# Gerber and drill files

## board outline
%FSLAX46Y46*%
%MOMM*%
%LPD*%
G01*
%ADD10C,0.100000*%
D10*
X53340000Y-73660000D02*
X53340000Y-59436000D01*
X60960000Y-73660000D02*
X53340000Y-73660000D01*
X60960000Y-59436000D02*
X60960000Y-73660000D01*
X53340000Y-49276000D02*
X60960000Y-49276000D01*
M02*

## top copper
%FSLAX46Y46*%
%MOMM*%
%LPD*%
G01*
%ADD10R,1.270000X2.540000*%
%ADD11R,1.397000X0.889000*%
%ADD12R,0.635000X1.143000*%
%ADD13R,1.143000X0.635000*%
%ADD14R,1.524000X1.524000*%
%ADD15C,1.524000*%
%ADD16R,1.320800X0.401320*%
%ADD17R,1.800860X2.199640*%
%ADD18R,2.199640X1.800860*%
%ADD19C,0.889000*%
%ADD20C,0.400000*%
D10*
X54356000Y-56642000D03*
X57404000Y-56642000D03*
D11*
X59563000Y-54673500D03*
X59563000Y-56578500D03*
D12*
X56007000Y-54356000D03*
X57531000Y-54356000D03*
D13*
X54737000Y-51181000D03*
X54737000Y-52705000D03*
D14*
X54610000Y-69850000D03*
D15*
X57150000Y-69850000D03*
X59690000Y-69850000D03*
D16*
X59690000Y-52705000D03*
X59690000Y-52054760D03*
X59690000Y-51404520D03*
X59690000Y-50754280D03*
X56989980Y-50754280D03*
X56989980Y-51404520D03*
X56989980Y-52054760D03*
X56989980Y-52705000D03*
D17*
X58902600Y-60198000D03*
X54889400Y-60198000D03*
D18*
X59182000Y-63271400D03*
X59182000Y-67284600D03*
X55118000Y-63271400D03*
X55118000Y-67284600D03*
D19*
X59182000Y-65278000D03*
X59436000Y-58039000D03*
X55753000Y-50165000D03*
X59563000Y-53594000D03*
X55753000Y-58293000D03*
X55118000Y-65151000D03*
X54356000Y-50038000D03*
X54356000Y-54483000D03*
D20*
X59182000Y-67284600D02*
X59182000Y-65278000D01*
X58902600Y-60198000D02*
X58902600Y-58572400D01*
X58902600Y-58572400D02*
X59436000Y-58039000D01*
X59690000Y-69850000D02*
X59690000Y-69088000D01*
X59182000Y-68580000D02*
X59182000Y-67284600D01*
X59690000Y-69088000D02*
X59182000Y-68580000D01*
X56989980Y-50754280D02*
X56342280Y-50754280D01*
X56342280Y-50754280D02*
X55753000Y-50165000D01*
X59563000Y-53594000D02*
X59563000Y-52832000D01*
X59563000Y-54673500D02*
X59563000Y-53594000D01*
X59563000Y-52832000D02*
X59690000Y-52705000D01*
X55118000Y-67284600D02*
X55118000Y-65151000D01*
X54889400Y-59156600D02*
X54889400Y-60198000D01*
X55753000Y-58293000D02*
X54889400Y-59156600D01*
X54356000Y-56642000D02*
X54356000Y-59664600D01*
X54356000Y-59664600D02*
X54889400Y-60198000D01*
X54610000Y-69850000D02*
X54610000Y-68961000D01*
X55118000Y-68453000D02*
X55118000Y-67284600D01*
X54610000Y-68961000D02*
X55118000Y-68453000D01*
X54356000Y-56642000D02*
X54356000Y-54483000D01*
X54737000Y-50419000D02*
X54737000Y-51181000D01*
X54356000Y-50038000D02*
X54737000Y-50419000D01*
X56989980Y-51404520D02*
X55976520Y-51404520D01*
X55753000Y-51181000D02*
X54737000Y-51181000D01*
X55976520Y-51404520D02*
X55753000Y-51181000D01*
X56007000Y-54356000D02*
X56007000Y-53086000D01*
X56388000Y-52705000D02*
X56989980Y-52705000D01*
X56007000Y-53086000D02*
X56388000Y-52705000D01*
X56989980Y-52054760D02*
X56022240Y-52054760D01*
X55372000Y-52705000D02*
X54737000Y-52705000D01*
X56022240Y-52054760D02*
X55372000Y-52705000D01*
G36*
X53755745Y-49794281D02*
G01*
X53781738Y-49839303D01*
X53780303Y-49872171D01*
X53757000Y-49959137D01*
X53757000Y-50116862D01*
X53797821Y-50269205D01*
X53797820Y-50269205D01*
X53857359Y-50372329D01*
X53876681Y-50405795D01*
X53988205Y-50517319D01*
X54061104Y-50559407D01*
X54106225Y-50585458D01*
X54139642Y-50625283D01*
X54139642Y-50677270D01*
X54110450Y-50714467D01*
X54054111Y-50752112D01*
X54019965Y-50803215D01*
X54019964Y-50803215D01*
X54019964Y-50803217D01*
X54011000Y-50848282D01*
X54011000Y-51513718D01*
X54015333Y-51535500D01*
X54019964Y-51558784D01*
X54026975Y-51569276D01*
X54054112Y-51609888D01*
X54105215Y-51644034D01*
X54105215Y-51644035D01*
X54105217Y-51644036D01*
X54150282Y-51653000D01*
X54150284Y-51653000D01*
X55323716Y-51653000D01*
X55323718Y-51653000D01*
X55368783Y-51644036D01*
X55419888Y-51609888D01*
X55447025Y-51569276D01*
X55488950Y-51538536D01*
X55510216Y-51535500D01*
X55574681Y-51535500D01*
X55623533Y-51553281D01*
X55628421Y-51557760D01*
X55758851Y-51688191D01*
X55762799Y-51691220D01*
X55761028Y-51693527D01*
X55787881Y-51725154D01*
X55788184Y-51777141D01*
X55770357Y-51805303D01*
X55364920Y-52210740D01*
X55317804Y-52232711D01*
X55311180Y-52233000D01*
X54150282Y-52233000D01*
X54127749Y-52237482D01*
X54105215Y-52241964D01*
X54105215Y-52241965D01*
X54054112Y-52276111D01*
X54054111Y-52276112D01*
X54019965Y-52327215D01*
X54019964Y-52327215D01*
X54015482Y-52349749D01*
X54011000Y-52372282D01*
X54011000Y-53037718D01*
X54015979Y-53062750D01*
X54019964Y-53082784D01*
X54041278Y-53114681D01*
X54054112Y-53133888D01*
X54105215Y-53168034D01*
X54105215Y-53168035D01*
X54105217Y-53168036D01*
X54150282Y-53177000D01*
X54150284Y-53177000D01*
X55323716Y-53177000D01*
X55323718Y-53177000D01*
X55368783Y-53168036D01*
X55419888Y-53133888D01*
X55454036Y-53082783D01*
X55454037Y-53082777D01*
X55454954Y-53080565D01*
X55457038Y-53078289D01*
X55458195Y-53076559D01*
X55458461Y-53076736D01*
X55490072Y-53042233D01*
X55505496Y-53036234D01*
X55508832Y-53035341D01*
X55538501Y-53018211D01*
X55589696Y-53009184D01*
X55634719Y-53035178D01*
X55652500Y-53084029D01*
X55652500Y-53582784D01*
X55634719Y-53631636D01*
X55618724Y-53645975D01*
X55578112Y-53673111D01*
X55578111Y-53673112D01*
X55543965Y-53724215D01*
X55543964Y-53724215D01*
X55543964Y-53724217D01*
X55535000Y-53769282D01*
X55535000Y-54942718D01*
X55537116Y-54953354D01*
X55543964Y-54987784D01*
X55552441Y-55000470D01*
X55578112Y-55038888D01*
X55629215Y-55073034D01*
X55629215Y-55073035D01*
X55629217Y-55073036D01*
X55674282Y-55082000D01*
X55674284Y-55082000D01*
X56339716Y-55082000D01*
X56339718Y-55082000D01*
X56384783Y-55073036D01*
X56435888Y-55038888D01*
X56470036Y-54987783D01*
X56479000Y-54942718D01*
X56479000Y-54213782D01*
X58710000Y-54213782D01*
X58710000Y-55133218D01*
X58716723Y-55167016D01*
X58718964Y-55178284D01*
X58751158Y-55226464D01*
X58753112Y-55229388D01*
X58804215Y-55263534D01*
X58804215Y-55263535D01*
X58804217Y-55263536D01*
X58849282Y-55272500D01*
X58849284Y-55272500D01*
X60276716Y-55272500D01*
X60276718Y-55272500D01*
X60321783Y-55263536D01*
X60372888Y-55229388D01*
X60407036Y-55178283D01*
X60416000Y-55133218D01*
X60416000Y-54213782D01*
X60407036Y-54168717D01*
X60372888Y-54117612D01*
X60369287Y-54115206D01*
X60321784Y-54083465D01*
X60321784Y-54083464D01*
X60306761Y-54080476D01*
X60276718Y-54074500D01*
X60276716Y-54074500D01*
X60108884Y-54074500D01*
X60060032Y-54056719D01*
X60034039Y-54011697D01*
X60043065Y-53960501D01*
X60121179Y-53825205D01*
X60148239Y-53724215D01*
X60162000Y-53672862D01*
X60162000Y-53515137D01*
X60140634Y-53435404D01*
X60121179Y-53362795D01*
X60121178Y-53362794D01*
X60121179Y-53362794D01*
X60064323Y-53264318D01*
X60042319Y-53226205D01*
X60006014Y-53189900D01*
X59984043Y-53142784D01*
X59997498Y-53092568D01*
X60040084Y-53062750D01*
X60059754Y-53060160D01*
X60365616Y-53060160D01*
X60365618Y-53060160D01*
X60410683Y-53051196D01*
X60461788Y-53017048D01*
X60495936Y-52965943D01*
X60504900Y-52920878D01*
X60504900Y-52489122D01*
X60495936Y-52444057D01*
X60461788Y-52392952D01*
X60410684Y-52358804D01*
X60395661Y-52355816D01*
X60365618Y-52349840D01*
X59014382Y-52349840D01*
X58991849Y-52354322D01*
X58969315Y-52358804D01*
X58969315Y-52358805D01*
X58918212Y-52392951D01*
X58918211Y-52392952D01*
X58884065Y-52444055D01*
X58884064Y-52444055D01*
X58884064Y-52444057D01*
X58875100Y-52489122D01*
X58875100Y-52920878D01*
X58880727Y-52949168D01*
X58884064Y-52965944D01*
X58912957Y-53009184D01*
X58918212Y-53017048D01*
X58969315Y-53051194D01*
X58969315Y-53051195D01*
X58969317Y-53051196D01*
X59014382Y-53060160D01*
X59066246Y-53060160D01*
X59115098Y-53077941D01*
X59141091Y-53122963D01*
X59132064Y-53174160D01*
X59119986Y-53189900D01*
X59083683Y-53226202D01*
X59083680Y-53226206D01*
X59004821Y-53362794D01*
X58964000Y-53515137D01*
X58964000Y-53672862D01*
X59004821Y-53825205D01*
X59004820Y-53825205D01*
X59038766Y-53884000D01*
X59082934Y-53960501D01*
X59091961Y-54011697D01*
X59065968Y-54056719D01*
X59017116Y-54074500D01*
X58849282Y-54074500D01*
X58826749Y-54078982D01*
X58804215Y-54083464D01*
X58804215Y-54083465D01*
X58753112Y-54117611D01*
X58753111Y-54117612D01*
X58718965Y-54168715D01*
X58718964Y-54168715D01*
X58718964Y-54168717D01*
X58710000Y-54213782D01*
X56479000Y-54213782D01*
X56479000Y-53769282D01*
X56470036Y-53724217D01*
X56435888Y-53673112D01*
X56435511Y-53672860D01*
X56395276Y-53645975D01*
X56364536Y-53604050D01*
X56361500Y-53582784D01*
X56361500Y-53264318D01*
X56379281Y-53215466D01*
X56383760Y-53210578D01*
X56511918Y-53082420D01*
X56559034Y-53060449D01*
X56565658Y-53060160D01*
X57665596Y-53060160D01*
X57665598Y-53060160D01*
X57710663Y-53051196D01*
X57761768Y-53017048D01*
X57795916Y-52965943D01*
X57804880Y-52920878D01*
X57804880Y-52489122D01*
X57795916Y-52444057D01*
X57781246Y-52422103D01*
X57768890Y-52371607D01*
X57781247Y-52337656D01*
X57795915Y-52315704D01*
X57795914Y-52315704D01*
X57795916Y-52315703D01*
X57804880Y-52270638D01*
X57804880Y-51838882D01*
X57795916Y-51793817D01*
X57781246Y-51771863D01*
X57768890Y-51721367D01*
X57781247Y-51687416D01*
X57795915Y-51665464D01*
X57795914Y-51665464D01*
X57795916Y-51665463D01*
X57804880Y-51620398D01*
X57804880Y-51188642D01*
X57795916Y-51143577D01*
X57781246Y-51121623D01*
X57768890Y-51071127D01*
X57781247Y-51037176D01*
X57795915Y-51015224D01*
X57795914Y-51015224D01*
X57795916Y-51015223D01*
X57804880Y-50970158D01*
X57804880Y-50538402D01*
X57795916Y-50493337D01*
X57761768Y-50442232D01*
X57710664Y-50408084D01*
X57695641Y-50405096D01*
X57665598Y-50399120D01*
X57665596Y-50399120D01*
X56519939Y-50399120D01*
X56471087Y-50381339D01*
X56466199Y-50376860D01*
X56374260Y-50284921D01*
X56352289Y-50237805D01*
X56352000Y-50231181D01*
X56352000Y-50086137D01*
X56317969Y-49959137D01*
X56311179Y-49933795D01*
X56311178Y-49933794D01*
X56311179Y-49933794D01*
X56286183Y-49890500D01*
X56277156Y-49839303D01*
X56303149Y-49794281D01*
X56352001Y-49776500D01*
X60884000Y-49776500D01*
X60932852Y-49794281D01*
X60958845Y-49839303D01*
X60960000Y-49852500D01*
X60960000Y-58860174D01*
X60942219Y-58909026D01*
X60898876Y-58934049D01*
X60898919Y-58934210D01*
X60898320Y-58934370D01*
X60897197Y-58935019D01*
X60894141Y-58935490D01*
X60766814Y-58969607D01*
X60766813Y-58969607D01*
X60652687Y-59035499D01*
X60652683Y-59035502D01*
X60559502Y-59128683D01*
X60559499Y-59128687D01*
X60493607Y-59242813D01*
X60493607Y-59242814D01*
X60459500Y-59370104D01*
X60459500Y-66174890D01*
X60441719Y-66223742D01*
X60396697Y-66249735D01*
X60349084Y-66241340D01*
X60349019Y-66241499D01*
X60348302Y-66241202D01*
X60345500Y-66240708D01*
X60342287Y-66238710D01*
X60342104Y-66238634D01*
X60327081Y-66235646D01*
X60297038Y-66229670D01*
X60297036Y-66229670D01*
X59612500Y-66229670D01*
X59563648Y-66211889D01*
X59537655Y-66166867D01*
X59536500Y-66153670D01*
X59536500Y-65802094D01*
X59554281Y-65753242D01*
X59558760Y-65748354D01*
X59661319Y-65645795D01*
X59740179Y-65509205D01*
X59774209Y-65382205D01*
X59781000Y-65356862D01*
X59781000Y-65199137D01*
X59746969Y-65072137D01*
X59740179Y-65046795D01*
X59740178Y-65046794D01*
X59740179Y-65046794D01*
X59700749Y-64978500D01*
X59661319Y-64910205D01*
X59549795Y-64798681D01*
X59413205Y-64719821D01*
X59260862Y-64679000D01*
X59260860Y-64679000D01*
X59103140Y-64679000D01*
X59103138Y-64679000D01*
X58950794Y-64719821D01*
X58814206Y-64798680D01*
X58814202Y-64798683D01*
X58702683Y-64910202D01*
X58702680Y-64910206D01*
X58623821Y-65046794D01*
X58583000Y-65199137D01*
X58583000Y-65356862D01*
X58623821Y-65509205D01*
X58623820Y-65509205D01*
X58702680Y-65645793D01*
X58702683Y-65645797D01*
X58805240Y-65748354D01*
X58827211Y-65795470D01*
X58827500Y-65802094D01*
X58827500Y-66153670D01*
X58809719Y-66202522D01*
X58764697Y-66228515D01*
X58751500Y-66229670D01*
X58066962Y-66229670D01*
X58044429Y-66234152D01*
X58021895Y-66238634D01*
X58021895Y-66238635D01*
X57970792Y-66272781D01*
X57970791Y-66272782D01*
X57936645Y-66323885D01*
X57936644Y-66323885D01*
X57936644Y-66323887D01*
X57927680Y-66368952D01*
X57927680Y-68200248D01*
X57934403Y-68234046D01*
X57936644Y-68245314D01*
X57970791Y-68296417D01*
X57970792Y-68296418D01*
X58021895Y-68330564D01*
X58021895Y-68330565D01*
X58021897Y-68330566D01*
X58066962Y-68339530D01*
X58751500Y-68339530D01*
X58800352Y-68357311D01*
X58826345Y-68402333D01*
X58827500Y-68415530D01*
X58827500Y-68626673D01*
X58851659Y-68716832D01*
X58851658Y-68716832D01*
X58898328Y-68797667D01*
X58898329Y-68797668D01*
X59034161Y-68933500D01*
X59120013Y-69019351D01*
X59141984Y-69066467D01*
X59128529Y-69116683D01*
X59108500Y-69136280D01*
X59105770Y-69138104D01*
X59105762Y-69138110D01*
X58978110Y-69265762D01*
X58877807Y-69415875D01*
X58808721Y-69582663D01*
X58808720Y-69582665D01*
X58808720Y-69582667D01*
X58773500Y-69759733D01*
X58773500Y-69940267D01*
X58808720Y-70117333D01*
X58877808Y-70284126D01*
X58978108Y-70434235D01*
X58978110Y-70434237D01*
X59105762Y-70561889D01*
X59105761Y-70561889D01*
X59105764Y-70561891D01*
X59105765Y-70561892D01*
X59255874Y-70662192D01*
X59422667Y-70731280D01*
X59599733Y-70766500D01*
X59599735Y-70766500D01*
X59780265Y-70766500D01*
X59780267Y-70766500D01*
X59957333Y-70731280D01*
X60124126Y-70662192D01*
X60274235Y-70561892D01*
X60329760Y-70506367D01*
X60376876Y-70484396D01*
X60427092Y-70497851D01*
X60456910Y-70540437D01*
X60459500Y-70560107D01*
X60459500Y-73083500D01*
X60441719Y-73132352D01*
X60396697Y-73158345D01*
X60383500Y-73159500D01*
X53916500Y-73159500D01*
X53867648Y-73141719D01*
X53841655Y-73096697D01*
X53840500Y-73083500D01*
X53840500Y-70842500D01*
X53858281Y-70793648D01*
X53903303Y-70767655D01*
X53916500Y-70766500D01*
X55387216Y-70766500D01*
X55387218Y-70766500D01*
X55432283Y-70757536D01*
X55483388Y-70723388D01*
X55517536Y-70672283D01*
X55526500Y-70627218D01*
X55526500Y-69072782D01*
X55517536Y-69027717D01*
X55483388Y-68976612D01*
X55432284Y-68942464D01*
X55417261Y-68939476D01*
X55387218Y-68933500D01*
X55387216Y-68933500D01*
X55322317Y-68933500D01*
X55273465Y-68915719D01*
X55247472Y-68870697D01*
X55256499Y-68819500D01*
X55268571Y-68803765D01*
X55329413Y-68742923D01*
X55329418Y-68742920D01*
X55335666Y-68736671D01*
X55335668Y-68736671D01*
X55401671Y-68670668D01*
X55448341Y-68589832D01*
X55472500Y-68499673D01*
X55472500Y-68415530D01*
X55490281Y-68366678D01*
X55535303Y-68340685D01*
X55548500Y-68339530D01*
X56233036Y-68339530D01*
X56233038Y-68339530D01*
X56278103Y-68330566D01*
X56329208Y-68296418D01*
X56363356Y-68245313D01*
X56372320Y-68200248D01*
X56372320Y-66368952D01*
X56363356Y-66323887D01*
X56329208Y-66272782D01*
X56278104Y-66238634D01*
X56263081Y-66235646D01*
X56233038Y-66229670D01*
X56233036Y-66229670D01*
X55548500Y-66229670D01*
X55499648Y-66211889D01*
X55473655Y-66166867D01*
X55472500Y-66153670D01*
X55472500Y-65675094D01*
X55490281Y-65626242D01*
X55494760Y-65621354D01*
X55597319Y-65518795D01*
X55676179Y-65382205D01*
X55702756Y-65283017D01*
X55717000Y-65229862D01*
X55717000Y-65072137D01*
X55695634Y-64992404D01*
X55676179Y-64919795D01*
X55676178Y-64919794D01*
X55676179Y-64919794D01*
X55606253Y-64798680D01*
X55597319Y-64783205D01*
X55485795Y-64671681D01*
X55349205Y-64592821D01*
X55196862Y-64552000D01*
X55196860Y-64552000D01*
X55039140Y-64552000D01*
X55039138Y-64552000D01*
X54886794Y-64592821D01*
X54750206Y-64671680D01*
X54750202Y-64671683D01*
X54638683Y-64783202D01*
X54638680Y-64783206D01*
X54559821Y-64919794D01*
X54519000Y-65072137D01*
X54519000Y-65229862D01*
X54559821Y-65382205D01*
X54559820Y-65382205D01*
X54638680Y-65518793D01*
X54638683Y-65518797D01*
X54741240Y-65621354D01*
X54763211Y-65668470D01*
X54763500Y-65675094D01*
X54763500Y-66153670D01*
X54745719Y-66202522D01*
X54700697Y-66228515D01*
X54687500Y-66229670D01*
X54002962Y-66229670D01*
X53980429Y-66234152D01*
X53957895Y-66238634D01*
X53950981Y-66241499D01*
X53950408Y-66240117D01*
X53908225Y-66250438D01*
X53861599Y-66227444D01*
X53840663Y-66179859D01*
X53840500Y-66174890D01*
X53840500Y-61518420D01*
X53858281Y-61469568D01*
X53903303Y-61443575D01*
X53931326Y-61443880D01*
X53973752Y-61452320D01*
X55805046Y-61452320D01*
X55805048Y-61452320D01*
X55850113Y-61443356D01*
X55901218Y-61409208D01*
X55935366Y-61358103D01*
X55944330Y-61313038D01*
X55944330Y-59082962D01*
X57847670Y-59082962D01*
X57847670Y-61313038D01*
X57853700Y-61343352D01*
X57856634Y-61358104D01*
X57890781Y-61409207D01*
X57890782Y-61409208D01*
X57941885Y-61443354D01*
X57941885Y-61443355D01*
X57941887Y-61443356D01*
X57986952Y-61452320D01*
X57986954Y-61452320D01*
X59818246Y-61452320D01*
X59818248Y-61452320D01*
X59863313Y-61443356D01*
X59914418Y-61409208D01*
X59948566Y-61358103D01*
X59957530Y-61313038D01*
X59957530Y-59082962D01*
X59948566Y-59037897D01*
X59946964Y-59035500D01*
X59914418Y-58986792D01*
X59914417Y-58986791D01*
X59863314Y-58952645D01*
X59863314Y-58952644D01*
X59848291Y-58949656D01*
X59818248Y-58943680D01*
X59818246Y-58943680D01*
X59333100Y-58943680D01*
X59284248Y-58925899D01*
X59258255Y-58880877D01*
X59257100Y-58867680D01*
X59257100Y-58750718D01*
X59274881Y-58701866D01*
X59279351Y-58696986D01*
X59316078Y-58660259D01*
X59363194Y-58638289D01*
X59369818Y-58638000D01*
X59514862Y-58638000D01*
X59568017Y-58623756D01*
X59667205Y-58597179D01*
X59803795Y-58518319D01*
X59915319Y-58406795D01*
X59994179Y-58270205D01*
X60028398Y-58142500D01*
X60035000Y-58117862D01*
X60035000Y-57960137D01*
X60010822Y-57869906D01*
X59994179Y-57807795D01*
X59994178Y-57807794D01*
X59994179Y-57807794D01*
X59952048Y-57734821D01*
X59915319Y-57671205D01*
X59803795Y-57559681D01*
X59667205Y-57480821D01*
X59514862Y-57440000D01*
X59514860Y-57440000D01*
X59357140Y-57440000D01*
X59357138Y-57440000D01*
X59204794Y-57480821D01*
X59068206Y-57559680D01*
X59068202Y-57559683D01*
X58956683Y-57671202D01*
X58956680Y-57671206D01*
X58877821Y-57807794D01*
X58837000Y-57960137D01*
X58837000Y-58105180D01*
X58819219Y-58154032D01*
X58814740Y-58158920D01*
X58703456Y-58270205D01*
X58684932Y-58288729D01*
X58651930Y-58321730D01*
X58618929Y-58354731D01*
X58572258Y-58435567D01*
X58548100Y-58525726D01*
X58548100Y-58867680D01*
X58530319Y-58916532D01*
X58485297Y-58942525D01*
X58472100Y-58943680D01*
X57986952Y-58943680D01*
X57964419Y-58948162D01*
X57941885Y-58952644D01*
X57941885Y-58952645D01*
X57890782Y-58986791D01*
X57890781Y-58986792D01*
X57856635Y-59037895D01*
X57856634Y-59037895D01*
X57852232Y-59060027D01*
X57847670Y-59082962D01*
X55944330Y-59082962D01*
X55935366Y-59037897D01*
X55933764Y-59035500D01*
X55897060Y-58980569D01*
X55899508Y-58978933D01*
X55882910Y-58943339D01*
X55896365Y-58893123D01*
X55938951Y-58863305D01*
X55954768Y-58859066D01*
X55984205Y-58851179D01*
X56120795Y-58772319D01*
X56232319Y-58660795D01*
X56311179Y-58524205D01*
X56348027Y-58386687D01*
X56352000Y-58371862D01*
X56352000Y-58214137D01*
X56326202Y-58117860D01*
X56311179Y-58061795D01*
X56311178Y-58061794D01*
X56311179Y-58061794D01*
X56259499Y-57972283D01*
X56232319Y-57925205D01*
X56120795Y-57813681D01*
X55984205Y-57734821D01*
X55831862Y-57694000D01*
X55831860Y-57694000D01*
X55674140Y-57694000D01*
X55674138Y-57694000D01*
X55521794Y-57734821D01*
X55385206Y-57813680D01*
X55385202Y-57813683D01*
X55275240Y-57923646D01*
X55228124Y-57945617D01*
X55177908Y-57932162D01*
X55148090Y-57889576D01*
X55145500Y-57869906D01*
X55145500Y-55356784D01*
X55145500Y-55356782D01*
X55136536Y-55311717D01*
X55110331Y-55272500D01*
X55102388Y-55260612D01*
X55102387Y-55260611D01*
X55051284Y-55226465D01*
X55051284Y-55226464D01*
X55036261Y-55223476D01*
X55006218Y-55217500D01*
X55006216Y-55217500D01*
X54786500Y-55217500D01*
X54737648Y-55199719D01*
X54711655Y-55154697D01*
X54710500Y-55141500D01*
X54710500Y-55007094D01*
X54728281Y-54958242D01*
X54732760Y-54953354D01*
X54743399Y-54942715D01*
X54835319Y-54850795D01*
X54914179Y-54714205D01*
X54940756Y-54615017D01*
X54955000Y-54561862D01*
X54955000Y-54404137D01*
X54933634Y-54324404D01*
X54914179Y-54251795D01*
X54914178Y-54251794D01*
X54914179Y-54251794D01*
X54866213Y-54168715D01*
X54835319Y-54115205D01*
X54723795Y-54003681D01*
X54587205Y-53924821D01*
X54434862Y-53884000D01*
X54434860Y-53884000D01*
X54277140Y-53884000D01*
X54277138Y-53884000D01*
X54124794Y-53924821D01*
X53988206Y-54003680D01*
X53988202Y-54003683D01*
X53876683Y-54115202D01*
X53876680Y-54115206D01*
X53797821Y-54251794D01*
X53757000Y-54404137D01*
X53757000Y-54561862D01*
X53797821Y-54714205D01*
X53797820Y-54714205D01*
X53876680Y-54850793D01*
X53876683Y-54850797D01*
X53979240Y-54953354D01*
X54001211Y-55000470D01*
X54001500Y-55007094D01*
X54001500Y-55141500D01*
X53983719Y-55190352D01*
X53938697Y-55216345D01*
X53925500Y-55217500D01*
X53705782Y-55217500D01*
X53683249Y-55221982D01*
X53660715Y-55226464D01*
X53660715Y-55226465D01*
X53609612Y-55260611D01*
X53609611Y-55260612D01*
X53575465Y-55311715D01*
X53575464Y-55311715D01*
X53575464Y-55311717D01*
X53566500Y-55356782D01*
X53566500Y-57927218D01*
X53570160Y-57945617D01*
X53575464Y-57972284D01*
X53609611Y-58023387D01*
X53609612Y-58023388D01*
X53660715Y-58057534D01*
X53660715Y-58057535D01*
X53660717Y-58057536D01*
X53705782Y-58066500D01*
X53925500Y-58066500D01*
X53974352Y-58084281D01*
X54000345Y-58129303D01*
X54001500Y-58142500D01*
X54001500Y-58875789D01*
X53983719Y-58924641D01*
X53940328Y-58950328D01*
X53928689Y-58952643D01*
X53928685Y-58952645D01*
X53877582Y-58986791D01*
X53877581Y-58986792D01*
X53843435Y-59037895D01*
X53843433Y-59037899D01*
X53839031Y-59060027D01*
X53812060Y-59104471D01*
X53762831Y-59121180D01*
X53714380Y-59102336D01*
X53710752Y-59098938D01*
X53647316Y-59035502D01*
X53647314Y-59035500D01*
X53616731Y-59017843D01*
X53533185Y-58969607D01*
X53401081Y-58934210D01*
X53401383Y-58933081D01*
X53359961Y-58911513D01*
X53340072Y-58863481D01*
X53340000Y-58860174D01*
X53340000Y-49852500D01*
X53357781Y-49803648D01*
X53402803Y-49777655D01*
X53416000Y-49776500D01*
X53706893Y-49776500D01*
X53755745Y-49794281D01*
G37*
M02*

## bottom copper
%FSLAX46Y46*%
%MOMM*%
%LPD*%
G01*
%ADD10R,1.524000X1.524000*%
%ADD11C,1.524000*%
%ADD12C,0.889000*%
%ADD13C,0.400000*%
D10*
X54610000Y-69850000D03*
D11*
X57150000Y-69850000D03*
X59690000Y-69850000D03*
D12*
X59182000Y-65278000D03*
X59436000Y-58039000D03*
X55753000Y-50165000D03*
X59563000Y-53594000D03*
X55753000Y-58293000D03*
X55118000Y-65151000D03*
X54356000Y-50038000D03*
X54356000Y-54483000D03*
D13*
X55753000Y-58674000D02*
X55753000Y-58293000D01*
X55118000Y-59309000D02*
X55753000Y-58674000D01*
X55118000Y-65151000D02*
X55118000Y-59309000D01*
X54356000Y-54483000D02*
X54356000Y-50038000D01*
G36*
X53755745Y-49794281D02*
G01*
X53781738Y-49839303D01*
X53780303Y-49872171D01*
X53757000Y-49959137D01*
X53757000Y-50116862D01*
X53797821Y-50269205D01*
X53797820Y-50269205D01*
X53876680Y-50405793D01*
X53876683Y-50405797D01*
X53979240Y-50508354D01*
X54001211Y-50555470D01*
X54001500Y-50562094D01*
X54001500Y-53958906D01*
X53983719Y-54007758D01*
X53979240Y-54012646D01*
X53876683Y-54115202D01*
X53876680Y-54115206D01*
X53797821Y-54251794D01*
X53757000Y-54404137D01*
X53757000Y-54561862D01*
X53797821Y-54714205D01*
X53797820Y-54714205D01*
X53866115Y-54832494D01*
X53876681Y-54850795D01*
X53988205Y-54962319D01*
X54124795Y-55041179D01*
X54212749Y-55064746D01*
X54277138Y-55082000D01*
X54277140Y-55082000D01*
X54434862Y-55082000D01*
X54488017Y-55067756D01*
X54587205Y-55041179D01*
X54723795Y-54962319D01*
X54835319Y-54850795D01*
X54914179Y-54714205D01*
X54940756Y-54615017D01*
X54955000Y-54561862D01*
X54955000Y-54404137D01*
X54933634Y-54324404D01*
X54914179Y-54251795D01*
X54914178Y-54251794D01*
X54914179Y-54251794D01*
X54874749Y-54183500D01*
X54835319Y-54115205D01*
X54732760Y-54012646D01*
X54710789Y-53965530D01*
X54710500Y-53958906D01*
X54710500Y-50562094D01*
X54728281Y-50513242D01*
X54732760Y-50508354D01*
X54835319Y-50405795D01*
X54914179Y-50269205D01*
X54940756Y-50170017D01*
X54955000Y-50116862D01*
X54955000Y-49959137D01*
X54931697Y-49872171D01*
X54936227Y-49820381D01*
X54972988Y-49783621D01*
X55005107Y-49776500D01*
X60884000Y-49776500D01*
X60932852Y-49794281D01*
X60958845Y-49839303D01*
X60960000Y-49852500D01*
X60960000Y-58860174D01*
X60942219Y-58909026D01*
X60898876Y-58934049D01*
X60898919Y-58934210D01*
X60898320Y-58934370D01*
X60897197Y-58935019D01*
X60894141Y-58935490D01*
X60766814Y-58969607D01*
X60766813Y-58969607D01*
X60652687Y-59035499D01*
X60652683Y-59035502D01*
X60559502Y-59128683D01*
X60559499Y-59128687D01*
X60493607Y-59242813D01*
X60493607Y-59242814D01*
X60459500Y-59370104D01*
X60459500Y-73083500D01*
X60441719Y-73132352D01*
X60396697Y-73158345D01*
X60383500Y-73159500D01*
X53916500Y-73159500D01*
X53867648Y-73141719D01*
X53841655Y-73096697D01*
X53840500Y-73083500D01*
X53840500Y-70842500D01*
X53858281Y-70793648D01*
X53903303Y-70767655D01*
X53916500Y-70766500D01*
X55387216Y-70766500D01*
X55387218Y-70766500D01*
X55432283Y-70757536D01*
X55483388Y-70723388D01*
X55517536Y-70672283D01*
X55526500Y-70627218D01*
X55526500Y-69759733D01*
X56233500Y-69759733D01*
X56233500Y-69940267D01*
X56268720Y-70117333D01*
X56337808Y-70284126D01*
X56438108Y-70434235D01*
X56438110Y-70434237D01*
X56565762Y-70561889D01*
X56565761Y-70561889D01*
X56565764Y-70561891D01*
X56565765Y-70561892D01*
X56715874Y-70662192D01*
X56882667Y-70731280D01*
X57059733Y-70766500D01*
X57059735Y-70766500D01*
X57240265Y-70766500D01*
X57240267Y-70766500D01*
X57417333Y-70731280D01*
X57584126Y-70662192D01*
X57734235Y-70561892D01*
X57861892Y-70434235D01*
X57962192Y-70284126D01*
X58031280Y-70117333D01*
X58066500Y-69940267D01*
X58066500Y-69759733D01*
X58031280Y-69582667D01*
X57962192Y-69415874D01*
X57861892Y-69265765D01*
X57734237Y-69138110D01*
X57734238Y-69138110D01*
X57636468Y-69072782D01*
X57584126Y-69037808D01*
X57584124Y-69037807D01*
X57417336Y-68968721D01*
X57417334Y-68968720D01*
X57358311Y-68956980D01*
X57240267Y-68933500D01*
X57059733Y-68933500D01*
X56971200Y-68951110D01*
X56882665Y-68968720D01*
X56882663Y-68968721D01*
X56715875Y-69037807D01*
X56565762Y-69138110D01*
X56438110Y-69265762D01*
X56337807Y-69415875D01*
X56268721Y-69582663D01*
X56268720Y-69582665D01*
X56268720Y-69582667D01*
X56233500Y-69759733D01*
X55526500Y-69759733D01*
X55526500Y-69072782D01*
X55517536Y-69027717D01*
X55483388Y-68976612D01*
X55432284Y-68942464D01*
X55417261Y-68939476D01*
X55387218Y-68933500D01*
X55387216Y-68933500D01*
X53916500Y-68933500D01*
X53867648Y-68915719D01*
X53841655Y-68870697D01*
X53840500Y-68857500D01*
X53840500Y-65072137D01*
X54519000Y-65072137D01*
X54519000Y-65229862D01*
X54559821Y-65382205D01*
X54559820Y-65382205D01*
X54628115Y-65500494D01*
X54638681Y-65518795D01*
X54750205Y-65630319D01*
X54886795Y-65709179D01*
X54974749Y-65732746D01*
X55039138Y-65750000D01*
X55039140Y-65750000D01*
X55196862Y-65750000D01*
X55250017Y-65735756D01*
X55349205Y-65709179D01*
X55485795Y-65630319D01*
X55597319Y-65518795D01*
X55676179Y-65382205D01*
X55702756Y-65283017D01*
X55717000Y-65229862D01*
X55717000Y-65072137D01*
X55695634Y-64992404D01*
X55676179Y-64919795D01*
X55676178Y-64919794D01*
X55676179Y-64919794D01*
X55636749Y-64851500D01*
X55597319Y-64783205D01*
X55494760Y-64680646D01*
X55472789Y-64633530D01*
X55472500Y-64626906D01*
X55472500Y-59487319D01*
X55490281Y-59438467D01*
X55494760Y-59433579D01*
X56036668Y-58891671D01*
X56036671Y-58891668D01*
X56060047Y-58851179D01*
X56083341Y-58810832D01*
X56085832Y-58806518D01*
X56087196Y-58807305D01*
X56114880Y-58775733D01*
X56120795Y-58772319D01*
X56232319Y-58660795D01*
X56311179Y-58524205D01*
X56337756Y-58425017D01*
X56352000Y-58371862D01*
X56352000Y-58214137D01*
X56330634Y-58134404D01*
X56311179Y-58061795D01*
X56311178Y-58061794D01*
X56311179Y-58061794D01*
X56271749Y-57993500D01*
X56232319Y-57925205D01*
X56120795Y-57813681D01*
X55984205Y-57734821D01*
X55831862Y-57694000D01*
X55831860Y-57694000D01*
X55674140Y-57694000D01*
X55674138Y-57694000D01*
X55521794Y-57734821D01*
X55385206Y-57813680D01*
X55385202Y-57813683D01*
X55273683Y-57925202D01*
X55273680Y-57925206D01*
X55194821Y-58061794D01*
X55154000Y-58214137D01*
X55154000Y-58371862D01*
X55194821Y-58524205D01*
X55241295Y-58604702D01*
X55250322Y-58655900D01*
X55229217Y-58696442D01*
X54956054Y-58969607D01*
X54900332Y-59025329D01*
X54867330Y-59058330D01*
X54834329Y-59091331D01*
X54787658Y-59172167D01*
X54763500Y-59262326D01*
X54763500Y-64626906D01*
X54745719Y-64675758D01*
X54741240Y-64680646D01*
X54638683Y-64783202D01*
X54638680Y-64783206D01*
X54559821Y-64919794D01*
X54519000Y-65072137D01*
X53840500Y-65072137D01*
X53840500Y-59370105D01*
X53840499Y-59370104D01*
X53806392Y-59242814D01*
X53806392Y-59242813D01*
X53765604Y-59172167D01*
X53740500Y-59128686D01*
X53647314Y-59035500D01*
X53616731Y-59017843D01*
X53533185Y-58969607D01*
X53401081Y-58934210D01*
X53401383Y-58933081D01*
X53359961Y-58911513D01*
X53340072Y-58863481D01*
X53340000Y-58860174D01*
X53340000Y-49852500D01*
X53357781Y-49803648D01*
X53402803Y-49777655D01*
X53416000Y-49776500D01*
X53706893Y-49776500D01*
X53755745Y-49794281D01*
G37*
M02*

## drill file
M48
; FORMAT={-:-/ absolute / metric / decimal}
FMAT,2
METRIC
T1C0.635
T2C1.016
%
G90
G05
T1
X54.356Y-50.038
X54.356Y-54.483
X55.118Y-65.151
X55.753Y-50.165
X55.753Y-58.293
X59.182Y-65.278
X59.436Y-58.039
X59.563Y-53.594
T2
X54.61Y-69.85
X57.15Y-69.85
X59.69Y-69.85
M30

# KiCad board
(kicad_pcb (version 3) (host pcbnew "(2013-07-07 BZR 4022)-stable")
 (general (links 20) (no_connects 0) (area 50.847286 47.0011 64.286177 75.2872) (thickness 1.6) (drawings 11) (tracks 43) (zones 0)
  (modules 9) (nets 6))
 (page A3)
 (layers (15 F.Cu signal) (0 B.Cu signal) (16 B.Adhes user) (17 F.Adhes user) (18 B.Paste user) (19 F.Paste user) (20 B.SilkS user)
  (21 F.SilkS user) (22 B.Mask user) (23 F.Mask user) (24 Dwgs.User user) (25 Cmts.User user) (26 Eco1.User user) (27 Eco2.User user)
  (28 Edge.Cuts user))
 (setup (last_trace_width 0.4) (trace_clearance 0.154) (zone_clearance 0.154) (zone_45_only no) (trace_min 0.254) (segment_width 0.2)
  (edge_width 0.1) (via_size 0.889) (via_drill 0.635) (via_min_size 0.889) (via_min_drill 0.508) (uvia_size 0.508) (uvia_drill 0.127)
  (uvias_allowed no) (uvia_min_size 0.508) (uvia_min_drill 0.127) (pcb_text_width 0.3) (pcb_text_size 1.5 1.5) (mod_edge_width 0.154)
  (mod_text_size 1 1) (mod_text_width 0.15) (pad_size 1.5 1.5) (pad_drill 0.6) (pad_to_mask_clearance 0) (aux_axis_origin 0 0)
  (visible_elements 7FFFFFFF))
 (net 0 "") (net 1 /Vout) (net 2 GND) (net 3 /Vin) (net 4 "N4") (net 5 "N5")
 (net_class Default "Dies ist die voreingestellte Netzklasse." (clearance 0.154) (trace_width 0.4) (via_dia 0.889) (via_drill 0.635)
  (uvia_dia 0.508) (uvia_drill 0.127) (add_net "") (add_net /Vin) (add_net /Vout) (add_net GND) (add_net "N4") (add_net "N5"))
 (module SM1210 (layer F.Cu) (at 55.88 56.642)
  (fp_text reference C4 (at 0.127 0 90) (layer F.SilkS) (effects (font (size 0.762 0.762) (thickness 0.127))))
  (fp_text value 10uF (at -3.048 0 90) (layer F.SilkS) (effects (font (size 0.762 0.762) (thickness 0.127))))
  (pad 1 smd rect (at -1.524 0) (size 1.27 2.54) (layers F.Cu F.Paste F.Mask) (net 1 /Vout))
  (pad 2 smd rect (at 1.524 0) (size 1.27 2.54) (layers F.Cu F.Paste F.Mask) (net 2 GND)))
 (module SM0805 (layer F.Cu) (at 59.563 55.626 270)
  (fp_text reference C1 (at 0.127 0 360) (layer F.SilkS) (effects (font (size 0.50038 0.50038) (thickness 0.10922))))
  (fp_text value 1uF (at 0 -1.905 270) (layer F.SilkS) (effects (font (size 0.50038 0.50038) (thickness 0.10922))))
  (pad 1 smd rect (at -0.9525 0 270) (size 0.889 1.397) (layers F.Cu F.Paste F.Mask) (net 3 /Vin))
  (pad 2 smd rect (at 0.9525 0 270) (size 0.889 1.397) (layers F.Cu F.Paste F.Mask) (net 2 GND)))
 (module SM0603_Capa (layer F.Cu) (at 56.769 54.356)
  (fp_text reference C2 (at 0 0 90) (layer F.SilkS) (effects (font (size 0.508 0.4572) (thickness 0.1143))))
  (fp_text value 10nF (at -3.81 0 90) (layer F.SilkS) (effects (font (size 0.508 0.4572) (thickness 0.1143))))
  (pad 1 smd rect (at -0.762 0) (size 0.635 1.143) (layers F.Cu F.Paste F.Mask) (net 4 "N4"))
  (pad 2 smd rect (at 0.762 0) (size 0.635 1.143) (layers F.Cu F.Paste F.Mask) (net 2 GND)))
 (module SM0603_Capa (layer F.Cu) (at 54.737 51.943 270)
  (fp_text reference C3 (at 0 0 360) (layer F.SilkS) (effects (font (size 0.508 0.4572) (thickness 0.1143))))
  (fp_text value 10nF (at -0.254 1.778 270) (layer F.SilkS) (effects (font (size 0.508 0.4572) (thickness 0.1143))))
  (pad 1 smd rect (at -0.762 0 270) (size 0.635 1.143) (layers F.Cu F.Paste F.Mask) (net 1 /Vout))
  (pad 2 smd rect (at 0.762 0 270) (size 0.635 1.143) (layers F.Cu F.Paste F.Mask) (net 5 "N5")))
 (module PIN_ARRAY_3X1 (layer F.Cu) (at 57.15 69.85)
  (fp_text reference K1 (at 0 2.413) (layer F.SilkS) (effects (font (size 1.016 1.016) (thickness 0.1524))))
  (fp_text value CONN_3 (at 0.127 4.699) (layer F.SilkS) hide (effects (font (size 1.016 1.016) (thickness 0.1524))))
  (pad 1 thru_hole rect (at -2.54 0) (size 1.524 1.524) (drill 1.016) (layers *.Cu *.Mask F.SilkS) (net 1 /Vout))
  (pad 2 thru_hole circle (at 0 0) (size 1.524 1.524) (drill 1.016) (layers *.Cu *.Mask F.SilkS) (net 2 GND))
  (pad 3 thru_hole circle (at 2.54 0) (size 1.524 1.524) (drill 1.016) (layers *.Cu *.Mask F.SilkS) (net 3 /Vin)))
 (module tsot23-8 (layer F.Cu) (at 59.69 52.705 90)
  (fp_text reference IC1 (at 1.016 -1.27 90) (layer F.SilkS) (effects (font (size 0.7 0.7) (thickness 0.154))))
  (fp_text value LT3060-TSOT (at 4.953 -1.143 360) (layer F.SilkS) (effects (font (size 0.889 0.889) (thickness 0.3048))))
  (pad 1 smd rect (at 0 0 90) (size 0.40132 1.3208) (layers F.Cu F.Paste F.Mask) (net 3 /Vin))
  (pad 2 smd rect (at 0.65024 0 90) (size 0.40132 1.3208) (layers F.Cu F.Paste F.Mask) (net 2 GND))
  (pad 3 smd rect (at 1.30048 0 90) (size 0.40132 1.3208) (layers F.Cu F.Paste F.Mask) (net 2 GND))
  (pad 4 smd rect (at 1.95072 0 90) (size 0.40132 1.3208) (layers F.Cu F.Paste F.Mask) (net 2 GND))
  (pad 5 smd rect (at 1.95072 -2.70002 270) (size 0.40132 1.3208) (layers F.Cu F.Paste F.Mask) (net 3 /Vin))
  (pad 6 smd rect (at 1.30048 -2.70002 270) (size 0.40132 1.3208) (layers F.Cu F.Paste F.Mask) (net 1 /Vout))
  (pad 7 smd rect (at 0.65024 -2.70002 270) (size 0.40132 1.3208) (layers F.Cu F.Paste F.Mask) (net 5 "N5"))
  (pad 8 smd rect (at 0 -2.70002 270) (size 0.40132 1.3208) (layers F.Cu F.Paste F.Mask) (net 4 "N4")))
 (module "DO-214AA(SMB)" (layer F.Cu) (at 56.896 60.198 180)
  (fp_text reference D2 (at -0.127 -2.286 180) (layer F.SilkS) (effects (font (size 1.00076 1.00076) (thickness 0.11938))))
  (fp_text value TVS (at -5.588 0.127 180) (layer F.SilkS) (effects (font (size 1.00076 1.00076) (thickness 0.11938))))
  (pad 1 smd rect (at -2.0066 0 180) (size 1.80086 2.19964) (layers F.Cu F.Paste F.Mask) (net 3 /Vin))
  (pad 2 smd rect (at 2.0066 0 180) (size 1.80086 2.19964) (layers F.Cu F.Paste F.Mask) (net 1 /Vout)))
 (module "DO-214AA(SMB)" (layer F.Cu) (at 59.182 65.278 270)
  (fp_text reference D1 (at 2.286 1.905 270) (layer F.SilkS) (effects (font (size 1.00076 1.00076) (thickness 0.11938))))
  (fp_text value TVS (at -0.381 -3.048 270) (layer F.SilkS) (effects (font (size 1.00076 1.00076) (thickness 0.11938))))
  (pad 1 smd rect (at -2.0066 0 270) (size 1.80086 2.19964) (layers F.Cu F.Paste F.Mask) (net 2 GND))
  (pad 2 smd rect (at 2.0066 0 270) (size 1.80086 2.19964) (layers F.Cu F.Paste F.Mask) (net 3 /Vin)))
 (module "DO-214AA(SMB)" (layer F.Cu) (at 55.118 65.278 270)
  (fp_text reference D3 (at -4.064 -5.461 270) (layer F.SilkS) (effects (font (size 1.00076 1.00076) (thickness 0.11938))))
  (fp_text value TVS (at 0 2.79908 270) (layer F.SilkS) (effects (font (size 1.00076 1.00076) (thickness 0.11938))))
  (pad 1 smd rect (at -2.0066 0 270) (size 1.80086 2.19964) (layers F.Cu F.Paste F.Mask) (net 2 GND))
  (pad 2 smd rect (at 2.0066 0 270) (size 1.80086 2.19964) (layers F.Cu F.Paste F.Mask) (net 1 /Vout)))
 (gr_line (start 53.34 73.66) (end 53.34 59.436) (angle 90) (layer Edge.Cuts) (width 0.1))
 (gr_line (start 60.96 73.66) (end 53.34 73.66) (angle 90) (layer Edge.Cuts) (width 0.1))
 (gr_line (start 60.96 59.436) (end 60.96 73.66) (angle 90) (layer Edge.Cuts) (width 0.1))
 (gr_line (start 53.34 49.276) (end 60.96 49.276) (angle 90) (layer Edge.Cuts) (width 0.1))
 (segment (start 59.182 67.2846) (end 59.182 65.278) (width 0.4) (layer F.Cu) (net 3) (status 400000))
 (via (at 59.182 65.278) (size 0.889) (layers F.Cu B.Cu) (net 3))
 (segment (start 58.9026 60.198) (end 58.9026 58.5724) (width 0.4) (layer F.Cu) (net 3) (status 400000))
 (via (at 59.436 58.039) (size 0.889) (layers F.Cu B.Cu) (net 3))
 (segment (start 58.9026 58.5724) (end 59.436 58.039) (width 0.4) (layer F.Cu) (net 3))
 (segment (start 59.69 69.85) (end 59.69 69.088) (width 0.4) (layer F.Cu) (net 3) (status C00000))
 (segment (start 59.182 68.58) (end 59.182 67.2846) (width 0.4) (layer F.Cu) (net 3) (status 800000))
 (segment (start 59.69 69.088) (end 59.182 68.58) (width 0.4) (layer F.Cu) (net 3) (status 400000))
 (segment (start 56.98998 50.75428) (end 56.34228 50.75428) (width 0.4) (layer F.Cu) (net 3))
 (via (at 55.753 50.165) (size 0.889) (layers F.Cu B.Cu) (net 3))
 (segment (start 56.34228 50.75428) (end 55.753 50.165) (width 0.4) (layer F.Cu) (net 3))
 (segment (start 59.563 53.594) (end 59.563 52.832) (width 0.4) (layer F.Cu) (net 3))
 (via (at 59.563 53.594) (size 0.889) (layers F.Cu B.Cu) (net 3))
 (segment (start 59.563 54.6735) (end 59.563 53.594) (width 0.4) (layer F.Cu) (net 3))
 (segment (start 59.563 52.832) (end 59.69 52.705) (width 0.4) (layer F.Cu) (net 3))
 (segment (start 55.118 67.2846) (end 55.118 65.151) (width 0.4) (layer F.Cu) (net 1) (status 400000))
 (segment (start 54.8894 59.1566) (end 54.8894 60.198) (width 0.4) (layer F.Cu) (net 1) (status C00000))
 (segment (start 55.753 58.293) (end 54.8894 59.1566) (width 0.4) (layer F.Cu) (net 1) (status 800000))
 (via (at 55.753 58.293) (size 0.889) (layers F.Cu B.Cu) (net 1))
 (segment (start 55.753 58.674) (end 55.753 58.293) (width 0.4) (layer B.Cu) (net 1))
 (segment (start 55.118 59.309) (end 55.753 58.674) (width 0.4) (layer B.Cu) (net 1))
 (segment (start 55.118 65.151) (end 55.118 59.309) (width 0.4) (layer B.Cu) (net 1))
 (via (at 55.118 65.151) (size 0.889) (layers F.Cu B.Cu) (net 1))
 (segment (start 54.356 56.642) (end 54.356 59.6646) (width 0.4) (layer F.Cu) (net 1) (status C00000))
 (segment (start 54.356 59.6646) (end 54.8894 60.198) (width 0.4) (layer F.Cu) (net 1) (status C00000))
 (segment (start 54.61 69.85) (end 54.61 68.961) (width 0.4) (layer F.Cu) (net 1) (status 400000))
 (segment (start 55.118 68.453) (end 55.118 67.2846) (width 0.4) (layer F.Cu) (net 1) (status 800000))
 (segment (start 54.61 68.961) (end 55.118 68.453) (width 0.4) (layer F.Cu) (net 1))
 (segment (start 54.356 56.642) (end 54.356 54.483) (width 0.4) (layer F.Cu) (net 1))
 (segment (start 54.737 50.419) (end 54.737 51.181) (width 0.4) (layer F.Cu) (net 1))
 (segment (start 54.356 50.038) (end 54.737 50.419) (width 0.4) (layer F.Cu) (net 1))
 (via (at 54.356 50.038) (size 0.889) (layers F.Cu B.Cu) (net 1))
 (segment (start 54.356 54.483) (end 54.356 50.038) (width 0.4) (layer B.Cu) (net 1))
 (via (at 54.356 54.483) (size 0.889) (layers F.Cu B.Cu) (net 1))
 (segment (start 56.98998 51.40452) (end 55.97652 51.40452) (width 0.4) (layer F.Cu) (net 1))
 (segment (start 55.753 51.181) (end 54.737 51.181) (width 0.4) (layer F.Cu) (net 1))
 (segment (start 55.97652 51.40452) (end 55.753 51.181) (width 0.4) (layer F.Cu) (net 1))
 (segment (start 56.007 54.356) (end 56.007 53.086) (width 0.4) (layer F.Cu) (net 4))
 (segment (start 56.388 52.705) (end 56.98998 52.705) (width 0.4) (layer F.Cu) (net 4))
 (segment (start 56.007 53.086) (end 56.388 52.705) (width 0.4) (layer F.Cu) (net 4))
 (segment (start 56.98998 52.05476) (end 56.02224 52.05476) (width 0.4) (layer F.Cu) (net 5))
 (segment (start 55.372 52.705) (end 54.737 52.705) (width 0.4) (layer F.Cu) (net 5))
 (segment (start 56.02224 52.05476) (end 55.372 52.705) (width 0.4) (layer F.Cu) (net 5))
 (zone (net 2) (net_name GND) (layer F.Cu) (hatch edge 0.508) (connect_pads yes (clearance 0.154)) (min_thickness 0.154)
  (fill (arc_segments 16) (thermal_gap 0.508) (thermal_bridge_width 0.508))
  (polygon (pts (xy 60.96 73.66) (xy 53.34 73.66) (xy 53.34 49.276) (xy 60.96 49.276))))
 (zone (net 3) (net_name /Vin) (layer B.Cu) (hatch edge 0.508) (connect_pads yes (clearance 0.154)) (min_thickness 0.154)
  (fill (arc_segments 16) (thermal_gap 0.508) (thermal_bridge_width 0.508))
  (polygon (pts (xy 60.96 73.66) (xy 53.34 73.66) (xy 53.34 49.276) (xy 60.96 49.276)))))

